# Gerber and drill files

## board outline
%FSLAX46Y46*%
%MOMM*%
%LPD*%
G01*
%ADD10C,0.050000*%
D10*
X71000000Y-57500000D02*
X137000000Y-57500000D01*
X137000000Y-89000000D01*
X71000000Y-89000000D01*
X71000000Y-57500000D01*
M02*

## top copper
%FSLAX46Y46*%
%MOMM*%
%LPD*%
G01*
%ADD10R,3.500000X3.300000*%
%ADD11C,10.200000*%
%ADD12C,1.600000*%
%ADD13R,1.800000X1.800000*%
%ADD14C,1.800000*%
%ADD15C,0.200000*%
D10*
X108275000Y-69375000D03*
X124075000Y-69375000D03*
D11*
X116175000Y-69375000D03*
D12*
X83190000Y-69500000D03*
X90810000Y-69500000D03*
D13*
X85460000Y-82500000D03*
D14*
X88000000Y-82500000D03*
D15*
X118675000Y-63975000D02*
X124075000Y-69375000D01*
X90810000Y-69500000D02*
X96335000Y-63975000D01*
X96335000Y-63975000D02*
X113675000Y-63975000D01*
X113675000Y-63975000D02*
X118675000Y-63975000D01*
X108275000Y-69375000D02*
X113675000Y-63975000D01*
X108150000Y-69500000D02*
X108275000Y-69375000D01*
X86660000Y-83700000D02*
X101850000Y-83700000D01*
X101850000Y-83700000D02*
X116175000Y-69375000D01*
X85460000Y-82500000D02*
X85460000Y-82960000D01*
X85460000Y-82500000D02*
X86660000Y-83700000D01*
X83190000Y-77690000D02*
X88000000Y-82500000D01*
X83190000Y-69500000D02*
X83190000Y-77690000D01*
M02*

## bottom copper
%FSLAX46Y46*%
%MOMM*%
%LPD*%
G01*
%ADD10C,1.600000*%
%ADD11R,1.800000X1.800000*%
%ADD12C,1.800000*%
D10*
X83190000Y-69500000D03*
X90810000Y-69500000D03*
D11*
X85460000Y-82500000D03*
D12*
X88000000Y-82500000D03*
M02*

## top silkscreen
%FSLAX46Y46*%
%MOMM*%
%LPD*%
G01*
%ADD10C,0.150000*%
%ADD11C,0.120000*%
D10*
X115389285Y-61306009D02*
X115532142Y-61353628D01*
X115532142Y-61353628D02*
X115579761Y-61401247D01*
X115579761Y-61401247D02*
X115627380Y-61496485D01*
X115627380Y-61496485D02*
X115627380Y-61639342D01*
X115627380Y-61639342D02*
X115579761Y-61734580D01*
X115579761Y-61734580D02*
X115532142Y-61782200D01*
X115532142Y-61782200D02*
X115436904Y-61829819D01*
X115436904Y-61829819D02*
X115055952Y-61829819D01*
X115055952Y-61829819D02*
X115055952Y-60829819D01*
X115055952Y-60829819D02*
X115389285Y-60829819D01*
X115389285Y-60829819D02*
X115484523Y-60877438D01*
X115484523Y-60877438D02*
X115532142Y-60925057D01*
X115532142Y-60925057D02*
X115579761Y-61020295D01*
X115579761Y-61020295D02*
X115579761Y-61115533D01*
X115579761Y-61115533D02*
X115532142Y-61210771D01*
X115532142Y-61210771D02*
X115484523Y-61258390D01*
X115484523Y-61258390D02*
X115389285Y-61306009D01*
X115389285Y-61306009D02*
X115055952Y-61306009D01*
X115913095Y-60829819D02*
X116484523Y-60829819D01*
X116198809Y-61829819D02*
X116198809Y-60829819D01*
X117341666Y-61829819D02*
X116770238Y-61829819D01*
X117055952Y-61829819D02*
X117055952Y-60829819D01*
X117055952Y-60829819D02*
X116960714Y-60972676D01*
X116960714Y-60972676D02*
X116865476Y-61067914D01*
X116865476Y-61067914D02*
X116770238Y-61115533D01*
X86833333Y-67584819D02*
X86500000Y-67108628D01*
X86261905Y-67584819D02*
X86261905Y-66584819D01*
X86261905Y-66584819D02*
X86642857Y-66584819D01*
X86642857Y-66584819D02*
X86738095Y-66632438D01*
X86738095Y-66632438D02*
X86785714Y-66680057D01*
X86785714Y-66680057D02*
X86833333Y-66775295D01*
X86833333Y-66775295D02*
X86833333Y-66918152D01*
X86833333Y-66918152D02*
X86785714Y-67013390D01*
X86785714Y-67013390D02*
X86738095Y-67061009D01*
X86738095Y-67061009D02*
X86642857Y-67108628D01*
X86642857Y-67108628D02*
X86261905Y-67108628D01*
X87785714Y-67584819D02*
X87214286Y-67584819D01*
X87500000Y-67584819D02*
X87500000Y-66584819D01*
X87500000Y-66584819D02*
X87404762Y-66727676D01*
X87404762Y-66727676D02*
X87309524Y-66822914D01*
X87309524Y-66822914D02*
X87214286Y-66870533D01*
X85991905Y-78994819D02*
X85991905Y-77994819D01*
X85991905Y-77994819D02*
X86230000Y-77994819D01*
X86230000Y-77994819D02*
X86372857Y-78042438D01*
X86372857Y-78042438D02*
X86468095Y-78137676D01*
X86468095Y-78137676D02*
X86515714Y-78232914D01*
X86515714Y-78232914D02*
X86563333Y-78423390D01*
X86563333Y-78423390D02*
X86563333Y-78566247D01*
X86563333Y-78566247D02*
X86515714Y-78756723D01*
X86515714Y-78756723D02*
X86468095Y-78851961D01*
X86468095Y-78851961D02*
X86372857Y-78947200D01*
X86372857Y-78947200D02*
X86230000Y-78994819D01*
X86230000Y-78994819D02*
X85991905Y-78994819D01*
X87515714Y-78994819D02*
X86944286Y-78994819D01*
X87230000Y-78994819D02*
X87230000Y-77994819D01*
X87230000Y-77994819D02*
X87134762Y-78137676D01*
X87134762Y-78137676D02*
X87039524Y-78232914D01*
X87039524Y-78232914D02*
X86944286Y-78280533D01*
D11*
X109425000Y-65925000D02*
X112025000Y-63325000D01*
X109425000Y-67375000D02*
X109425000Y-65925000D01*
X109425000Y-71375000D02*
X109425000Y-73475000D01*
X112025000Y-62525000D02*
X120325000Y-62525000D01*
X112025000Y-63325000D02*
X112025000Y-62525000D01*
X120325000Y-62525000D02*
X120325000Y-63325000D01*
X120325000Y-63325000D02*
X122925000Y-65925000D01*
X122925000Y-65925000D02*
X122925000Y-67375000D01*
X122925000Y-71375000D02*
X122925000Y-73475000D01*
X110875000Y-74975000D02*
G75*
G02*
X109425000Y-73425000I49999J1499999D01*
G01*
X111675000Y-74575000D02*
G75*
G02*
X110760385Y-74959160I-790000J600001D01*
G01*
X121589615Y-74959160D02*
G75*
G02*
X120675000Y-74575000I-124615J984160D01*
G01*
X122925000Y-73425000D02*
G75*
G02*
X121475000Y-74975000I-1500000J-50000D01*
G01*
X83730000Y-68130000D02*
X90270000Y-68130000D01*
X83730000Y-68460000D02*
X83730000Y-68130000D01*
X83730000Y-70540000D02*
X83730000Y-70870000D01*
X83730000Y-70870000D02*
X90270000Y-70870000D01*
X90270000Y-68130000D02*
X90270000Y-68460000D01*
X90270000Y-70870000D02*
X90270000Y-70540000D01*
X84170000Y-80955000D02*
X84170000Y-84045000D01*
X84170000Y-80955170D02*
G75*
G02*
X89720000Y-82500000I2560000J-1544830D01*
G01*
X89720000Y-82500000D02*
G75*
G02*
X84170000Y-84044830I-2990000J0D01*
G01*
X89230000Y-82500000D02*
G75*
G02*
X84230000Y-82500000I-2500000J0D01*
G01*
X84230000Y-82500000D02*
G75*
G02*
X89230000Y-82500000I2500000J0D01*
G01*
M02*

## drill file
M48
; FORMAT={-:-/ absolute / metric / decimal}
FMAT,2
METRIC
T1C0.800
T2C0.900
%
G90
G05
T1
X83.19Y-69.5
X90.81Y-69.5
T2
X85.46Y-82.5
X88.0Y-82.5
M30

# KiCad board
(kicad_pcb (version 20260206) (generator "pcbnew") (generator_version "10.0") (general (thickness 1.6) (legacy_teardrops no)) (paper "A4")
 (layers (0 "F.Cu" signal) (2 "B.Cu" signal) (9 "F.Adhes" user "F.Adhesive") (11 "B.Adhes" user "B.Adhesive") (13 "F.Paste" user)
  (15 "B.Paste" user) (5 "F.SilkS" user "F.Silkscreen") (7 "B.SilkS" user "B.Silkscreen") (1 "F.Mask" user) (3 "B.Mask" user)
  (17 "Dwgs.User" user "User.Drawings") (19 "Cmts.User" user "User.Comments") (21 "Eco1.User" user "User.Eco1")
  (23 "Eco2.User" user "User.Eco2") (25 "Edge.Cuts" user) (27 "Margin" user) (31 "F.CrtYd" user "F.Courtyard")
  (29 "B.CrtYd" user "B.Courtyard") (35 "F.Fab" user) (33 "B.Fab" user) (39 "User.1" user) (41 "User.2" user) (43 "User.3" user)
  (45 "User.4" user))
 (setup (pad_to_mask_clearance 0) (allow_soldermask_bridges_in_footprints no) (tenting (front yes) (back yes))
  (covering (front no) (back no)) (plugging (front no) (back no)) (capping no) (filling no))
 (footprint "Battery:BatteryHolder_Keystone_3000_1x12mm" (layer "F.Cu") (at 116.175 69.375)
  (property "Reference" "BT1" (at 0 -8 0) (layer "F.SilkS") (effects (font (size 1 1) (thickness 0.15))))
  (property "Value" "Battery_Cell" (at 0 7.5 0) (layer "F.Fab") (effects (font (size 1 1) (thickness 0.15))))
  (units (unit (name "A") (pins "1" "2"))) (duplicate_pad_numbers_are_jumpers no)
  (fp_line (start -6.75 -3.45) (end -4.15 -6.05) (stroke (width 0.12) (type solid)) (layer "F.SilkS"))
  (fp_line (start -6.75 -2) (end -6.75 -3.45) (stroke (width 0.12) (type solid)) (layer "F.SilkS"))
  (fp_line (start -6.75 2) (end -6.75 4.1) (stroke (width 0.12) (type solid)) (layer "F.SilkS"))
  (fp_line (start -4.15 -6.85) (end 4.15 -6.85) (stroke (width 0.12) (type solid)) (layer "F.SilkS"))
  (fp_line (start -4.15 -6.05) (end -4.15 -6.85) (stroke (width 0.12) (type solid)) (layer "F.SilkS"))
  (fp_line (start 4.15 -6.85) (end 4.15 -6.05) (stroke (width 0.12) (type solid)) (layer "F.SilkS"))
  (fp_line (start 4.15 -6.05) (end 6.75 -3.45) (stroke (width 0.12) (type solid)) (layer "F.SilkS"))
  (fp_line (start 6.75 -3.45) (end 6.75 -2) (stroke (width 0.12) (type solid)) (layer "F.SilkS"))
  (fp_line (start 6.75 2) (end 6.75 4.1) (stroke (width 0.12) (type solid)) (layer "F.SilkS"))
  (fp_arc (start -5.3 5.6) (mid -6.346016 5.125305) (end -6.75 4.05) (stroke (width 0.12) (type solid)) (layer "F.SilkS"))
  (fp_arc (start -4.5 5.2) (mid -4.90584 5.514615) (end -5.414615 5.58416) (stroke (width 0.12) (type solid)) (layer "F.SilkS"))
  (fp_arc (start 5.414615 5.58416) (mid 4.90584 5.514615) (end 4.5 5.2) (stroke (width 0.12) (type solid)) (layer "F.SilkS"))
  (fp_arc (start 6.75 4.05) (mid 6.346016 5.125305) (end 5.3 5.6) (stroke (width 0.12) (type solid)) (layer "F.SilkS"))
  (pad "1" smd rect (at -7.9 0) (size 3.5 3.3) (layers "F.Cu" "F.Mask" "F.Paste") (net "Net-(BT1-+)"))
  (pad "1" smd rect (at 7.9 0) (size 3.5 3.3) (layers "F.Cu" "F.Mask" "F.Paste") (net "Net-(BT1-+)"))
  (pad "2" smd circle (at 0 0) (size 10.2 10.2) (layers "F.Cu" "F.Mask") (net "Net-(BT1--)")))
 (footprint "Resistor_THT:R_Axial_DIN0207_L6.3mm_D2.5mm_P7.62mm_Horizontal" (layer "F.Cu") (at 83.19 69.5)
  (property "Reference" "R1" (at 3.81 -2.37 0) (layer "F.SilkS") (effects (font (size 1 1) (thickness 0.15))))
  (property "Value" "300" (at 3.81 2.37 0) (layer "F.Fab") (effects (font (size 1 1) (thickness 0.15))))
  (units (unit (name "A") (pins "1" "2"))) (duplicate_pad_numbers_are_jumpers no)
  (fp_line (start 0.54 -1.37) (end 7.08 -1.37) (stroke (width 0.12) (type solid)) (layer "F.SilkS"))
  (fp_line (start 0.54 -1.04) (end 0.54 -1.37) (stroke (width 0.12) (type solid)) (layer "F.SilkS"))
  (fp_line (start 0.54 1.04) (end 0.54 1.37) (stroke (width 0.12) (type solid)) (layer "F.SilkS"))
  (fp_line (start 0.54 1.37) (end 7.08 1.37) (stroke (width 0.12) (type solid)) (layer "F.SilkS"))
  (fp_line (start 7.08 -1.37) (end 7.08 -1.04) (stroke (width 0.12) (type solid)) (layer "F.SilkS"))
  (fp_line (start 7.08 1.37) (end 7.08 1.04) (stroke (width 0.12) (type solid)) (layer "F.SilkS"))
  (pad "1" thru_hole circle (at 0 0) (size 1.6 1.6) (drill 0.8) (layers "*.Cu" "*.Mask") (remove_unused_layers no) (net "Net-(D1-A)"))
  (pad "2" thru_hole circle (at 7.62 0) (size 1.6 1.6) (drill 0.8) (layers "*.Cu" "*.Mask") (remove_unused_layers no) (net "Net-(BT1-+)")))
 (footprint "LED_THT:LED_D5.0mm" (layer "F.Cu") (at 85.46 82.5)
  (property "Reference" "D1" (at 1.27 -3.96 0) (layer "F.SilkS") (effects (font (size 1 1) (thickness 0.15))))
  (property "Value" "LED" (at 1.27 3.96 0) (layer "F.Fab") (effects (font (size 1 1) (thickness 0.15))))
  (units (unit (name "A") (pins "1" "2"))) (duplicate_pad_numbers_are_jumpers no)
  (fp_line (start -1.29 -1.545) (end -1.29 1.545) (stroke (width 0.12) (type solid)) (layer "F.SilkS"))
  (fp_arc (start -1.29 -1.54483) (mid 2.071779 -2.880495) (end 4.26 0) (stroke (width 0.12) (type solid)) (layer "F.SilkS"))
  (fp_arc (start 4.26 0) (mid 2.071779 2.880495) (end -1.29 1.54483) (stroke (width 0.12) (type solid)) (layer "F.SilkS"))
  (fp_circle (center 1.27 0) (end 3.77 0) (stroke (width 0.12) (type solid)) (fill no) (layer "F.SilkS"))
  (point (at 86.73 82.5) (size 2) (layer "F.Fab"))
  (pad "1" thru_hole rect (at 0 0) (size 1.8 1.8) (drill 0.9) (layers "*.Cu" "*.Mask") (remove_unused_layers no) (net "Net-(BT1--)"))
  (pad "2" thru_hole circle (at 2.54 0) (size 1.8 1.8) (drill 0.9) (layers "*.Cu" "*.Mask") (remove_unused_layers no) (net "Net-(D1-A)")))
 (gr_rect (start 71 57.5) (end 137 89) (stroke (width 0.05) (type default)) (fill no) (layer "Edge.Cuts"))
 (segment (start 118.675 63.975) (end 124.075 69.375) (width 0.2) (layer "F.Cu") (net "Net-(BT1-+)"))
 (segment (start 90.81 69.5) (end 96.335 63.975) (width 0.2) (layer "F.Cu") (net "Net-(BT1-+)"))
 (segment (start 96.335 63.975) (end 113.675 63.975) (width 0.2) (layer "F.Cu") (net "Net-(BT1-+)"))
 (segment (start 113.675 63.975) (end 118.675 63.975) (width 0.2) (layer "F.Cu") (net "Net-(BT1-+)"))
 (segment (start 108.275 69.375) (end 113.675 63.975) (width 0.2) (layer "F.Cu") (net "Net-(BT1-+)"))
 (segment (start 108.15 69.5) (end 108.275 69.375) (width 0.2) (layer "F.Cu") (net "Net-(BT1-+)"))
 (segment (start 86.66 83.7) (end 101.85 83.7) (width 0.2) (layer "F.Cu") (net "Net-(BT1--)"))
 (segment (start 101.85 83.7) (end 116.175 69.375) (width 0.2) (layer "F.Cu") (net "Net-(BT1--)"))
 (segment (start 85.46 82.5) (end 85.46 82.96) (width 0.2) (layer "F.Cu") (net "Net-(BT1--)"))
 (segment (start 85.46 82.5) (end 86.66 83.7) (width 0.2) (layer "F.Cu") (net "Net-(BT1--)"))
 (segment (start 83.19 77.69) (end 88 82.5) (width 0.2) (layer "F.Cu") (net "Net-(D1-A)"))
 (segment (start 83.19 69.5) (end 83.19 77.69) (width 0.2) (layer "F.Cu") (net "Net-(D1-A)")))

